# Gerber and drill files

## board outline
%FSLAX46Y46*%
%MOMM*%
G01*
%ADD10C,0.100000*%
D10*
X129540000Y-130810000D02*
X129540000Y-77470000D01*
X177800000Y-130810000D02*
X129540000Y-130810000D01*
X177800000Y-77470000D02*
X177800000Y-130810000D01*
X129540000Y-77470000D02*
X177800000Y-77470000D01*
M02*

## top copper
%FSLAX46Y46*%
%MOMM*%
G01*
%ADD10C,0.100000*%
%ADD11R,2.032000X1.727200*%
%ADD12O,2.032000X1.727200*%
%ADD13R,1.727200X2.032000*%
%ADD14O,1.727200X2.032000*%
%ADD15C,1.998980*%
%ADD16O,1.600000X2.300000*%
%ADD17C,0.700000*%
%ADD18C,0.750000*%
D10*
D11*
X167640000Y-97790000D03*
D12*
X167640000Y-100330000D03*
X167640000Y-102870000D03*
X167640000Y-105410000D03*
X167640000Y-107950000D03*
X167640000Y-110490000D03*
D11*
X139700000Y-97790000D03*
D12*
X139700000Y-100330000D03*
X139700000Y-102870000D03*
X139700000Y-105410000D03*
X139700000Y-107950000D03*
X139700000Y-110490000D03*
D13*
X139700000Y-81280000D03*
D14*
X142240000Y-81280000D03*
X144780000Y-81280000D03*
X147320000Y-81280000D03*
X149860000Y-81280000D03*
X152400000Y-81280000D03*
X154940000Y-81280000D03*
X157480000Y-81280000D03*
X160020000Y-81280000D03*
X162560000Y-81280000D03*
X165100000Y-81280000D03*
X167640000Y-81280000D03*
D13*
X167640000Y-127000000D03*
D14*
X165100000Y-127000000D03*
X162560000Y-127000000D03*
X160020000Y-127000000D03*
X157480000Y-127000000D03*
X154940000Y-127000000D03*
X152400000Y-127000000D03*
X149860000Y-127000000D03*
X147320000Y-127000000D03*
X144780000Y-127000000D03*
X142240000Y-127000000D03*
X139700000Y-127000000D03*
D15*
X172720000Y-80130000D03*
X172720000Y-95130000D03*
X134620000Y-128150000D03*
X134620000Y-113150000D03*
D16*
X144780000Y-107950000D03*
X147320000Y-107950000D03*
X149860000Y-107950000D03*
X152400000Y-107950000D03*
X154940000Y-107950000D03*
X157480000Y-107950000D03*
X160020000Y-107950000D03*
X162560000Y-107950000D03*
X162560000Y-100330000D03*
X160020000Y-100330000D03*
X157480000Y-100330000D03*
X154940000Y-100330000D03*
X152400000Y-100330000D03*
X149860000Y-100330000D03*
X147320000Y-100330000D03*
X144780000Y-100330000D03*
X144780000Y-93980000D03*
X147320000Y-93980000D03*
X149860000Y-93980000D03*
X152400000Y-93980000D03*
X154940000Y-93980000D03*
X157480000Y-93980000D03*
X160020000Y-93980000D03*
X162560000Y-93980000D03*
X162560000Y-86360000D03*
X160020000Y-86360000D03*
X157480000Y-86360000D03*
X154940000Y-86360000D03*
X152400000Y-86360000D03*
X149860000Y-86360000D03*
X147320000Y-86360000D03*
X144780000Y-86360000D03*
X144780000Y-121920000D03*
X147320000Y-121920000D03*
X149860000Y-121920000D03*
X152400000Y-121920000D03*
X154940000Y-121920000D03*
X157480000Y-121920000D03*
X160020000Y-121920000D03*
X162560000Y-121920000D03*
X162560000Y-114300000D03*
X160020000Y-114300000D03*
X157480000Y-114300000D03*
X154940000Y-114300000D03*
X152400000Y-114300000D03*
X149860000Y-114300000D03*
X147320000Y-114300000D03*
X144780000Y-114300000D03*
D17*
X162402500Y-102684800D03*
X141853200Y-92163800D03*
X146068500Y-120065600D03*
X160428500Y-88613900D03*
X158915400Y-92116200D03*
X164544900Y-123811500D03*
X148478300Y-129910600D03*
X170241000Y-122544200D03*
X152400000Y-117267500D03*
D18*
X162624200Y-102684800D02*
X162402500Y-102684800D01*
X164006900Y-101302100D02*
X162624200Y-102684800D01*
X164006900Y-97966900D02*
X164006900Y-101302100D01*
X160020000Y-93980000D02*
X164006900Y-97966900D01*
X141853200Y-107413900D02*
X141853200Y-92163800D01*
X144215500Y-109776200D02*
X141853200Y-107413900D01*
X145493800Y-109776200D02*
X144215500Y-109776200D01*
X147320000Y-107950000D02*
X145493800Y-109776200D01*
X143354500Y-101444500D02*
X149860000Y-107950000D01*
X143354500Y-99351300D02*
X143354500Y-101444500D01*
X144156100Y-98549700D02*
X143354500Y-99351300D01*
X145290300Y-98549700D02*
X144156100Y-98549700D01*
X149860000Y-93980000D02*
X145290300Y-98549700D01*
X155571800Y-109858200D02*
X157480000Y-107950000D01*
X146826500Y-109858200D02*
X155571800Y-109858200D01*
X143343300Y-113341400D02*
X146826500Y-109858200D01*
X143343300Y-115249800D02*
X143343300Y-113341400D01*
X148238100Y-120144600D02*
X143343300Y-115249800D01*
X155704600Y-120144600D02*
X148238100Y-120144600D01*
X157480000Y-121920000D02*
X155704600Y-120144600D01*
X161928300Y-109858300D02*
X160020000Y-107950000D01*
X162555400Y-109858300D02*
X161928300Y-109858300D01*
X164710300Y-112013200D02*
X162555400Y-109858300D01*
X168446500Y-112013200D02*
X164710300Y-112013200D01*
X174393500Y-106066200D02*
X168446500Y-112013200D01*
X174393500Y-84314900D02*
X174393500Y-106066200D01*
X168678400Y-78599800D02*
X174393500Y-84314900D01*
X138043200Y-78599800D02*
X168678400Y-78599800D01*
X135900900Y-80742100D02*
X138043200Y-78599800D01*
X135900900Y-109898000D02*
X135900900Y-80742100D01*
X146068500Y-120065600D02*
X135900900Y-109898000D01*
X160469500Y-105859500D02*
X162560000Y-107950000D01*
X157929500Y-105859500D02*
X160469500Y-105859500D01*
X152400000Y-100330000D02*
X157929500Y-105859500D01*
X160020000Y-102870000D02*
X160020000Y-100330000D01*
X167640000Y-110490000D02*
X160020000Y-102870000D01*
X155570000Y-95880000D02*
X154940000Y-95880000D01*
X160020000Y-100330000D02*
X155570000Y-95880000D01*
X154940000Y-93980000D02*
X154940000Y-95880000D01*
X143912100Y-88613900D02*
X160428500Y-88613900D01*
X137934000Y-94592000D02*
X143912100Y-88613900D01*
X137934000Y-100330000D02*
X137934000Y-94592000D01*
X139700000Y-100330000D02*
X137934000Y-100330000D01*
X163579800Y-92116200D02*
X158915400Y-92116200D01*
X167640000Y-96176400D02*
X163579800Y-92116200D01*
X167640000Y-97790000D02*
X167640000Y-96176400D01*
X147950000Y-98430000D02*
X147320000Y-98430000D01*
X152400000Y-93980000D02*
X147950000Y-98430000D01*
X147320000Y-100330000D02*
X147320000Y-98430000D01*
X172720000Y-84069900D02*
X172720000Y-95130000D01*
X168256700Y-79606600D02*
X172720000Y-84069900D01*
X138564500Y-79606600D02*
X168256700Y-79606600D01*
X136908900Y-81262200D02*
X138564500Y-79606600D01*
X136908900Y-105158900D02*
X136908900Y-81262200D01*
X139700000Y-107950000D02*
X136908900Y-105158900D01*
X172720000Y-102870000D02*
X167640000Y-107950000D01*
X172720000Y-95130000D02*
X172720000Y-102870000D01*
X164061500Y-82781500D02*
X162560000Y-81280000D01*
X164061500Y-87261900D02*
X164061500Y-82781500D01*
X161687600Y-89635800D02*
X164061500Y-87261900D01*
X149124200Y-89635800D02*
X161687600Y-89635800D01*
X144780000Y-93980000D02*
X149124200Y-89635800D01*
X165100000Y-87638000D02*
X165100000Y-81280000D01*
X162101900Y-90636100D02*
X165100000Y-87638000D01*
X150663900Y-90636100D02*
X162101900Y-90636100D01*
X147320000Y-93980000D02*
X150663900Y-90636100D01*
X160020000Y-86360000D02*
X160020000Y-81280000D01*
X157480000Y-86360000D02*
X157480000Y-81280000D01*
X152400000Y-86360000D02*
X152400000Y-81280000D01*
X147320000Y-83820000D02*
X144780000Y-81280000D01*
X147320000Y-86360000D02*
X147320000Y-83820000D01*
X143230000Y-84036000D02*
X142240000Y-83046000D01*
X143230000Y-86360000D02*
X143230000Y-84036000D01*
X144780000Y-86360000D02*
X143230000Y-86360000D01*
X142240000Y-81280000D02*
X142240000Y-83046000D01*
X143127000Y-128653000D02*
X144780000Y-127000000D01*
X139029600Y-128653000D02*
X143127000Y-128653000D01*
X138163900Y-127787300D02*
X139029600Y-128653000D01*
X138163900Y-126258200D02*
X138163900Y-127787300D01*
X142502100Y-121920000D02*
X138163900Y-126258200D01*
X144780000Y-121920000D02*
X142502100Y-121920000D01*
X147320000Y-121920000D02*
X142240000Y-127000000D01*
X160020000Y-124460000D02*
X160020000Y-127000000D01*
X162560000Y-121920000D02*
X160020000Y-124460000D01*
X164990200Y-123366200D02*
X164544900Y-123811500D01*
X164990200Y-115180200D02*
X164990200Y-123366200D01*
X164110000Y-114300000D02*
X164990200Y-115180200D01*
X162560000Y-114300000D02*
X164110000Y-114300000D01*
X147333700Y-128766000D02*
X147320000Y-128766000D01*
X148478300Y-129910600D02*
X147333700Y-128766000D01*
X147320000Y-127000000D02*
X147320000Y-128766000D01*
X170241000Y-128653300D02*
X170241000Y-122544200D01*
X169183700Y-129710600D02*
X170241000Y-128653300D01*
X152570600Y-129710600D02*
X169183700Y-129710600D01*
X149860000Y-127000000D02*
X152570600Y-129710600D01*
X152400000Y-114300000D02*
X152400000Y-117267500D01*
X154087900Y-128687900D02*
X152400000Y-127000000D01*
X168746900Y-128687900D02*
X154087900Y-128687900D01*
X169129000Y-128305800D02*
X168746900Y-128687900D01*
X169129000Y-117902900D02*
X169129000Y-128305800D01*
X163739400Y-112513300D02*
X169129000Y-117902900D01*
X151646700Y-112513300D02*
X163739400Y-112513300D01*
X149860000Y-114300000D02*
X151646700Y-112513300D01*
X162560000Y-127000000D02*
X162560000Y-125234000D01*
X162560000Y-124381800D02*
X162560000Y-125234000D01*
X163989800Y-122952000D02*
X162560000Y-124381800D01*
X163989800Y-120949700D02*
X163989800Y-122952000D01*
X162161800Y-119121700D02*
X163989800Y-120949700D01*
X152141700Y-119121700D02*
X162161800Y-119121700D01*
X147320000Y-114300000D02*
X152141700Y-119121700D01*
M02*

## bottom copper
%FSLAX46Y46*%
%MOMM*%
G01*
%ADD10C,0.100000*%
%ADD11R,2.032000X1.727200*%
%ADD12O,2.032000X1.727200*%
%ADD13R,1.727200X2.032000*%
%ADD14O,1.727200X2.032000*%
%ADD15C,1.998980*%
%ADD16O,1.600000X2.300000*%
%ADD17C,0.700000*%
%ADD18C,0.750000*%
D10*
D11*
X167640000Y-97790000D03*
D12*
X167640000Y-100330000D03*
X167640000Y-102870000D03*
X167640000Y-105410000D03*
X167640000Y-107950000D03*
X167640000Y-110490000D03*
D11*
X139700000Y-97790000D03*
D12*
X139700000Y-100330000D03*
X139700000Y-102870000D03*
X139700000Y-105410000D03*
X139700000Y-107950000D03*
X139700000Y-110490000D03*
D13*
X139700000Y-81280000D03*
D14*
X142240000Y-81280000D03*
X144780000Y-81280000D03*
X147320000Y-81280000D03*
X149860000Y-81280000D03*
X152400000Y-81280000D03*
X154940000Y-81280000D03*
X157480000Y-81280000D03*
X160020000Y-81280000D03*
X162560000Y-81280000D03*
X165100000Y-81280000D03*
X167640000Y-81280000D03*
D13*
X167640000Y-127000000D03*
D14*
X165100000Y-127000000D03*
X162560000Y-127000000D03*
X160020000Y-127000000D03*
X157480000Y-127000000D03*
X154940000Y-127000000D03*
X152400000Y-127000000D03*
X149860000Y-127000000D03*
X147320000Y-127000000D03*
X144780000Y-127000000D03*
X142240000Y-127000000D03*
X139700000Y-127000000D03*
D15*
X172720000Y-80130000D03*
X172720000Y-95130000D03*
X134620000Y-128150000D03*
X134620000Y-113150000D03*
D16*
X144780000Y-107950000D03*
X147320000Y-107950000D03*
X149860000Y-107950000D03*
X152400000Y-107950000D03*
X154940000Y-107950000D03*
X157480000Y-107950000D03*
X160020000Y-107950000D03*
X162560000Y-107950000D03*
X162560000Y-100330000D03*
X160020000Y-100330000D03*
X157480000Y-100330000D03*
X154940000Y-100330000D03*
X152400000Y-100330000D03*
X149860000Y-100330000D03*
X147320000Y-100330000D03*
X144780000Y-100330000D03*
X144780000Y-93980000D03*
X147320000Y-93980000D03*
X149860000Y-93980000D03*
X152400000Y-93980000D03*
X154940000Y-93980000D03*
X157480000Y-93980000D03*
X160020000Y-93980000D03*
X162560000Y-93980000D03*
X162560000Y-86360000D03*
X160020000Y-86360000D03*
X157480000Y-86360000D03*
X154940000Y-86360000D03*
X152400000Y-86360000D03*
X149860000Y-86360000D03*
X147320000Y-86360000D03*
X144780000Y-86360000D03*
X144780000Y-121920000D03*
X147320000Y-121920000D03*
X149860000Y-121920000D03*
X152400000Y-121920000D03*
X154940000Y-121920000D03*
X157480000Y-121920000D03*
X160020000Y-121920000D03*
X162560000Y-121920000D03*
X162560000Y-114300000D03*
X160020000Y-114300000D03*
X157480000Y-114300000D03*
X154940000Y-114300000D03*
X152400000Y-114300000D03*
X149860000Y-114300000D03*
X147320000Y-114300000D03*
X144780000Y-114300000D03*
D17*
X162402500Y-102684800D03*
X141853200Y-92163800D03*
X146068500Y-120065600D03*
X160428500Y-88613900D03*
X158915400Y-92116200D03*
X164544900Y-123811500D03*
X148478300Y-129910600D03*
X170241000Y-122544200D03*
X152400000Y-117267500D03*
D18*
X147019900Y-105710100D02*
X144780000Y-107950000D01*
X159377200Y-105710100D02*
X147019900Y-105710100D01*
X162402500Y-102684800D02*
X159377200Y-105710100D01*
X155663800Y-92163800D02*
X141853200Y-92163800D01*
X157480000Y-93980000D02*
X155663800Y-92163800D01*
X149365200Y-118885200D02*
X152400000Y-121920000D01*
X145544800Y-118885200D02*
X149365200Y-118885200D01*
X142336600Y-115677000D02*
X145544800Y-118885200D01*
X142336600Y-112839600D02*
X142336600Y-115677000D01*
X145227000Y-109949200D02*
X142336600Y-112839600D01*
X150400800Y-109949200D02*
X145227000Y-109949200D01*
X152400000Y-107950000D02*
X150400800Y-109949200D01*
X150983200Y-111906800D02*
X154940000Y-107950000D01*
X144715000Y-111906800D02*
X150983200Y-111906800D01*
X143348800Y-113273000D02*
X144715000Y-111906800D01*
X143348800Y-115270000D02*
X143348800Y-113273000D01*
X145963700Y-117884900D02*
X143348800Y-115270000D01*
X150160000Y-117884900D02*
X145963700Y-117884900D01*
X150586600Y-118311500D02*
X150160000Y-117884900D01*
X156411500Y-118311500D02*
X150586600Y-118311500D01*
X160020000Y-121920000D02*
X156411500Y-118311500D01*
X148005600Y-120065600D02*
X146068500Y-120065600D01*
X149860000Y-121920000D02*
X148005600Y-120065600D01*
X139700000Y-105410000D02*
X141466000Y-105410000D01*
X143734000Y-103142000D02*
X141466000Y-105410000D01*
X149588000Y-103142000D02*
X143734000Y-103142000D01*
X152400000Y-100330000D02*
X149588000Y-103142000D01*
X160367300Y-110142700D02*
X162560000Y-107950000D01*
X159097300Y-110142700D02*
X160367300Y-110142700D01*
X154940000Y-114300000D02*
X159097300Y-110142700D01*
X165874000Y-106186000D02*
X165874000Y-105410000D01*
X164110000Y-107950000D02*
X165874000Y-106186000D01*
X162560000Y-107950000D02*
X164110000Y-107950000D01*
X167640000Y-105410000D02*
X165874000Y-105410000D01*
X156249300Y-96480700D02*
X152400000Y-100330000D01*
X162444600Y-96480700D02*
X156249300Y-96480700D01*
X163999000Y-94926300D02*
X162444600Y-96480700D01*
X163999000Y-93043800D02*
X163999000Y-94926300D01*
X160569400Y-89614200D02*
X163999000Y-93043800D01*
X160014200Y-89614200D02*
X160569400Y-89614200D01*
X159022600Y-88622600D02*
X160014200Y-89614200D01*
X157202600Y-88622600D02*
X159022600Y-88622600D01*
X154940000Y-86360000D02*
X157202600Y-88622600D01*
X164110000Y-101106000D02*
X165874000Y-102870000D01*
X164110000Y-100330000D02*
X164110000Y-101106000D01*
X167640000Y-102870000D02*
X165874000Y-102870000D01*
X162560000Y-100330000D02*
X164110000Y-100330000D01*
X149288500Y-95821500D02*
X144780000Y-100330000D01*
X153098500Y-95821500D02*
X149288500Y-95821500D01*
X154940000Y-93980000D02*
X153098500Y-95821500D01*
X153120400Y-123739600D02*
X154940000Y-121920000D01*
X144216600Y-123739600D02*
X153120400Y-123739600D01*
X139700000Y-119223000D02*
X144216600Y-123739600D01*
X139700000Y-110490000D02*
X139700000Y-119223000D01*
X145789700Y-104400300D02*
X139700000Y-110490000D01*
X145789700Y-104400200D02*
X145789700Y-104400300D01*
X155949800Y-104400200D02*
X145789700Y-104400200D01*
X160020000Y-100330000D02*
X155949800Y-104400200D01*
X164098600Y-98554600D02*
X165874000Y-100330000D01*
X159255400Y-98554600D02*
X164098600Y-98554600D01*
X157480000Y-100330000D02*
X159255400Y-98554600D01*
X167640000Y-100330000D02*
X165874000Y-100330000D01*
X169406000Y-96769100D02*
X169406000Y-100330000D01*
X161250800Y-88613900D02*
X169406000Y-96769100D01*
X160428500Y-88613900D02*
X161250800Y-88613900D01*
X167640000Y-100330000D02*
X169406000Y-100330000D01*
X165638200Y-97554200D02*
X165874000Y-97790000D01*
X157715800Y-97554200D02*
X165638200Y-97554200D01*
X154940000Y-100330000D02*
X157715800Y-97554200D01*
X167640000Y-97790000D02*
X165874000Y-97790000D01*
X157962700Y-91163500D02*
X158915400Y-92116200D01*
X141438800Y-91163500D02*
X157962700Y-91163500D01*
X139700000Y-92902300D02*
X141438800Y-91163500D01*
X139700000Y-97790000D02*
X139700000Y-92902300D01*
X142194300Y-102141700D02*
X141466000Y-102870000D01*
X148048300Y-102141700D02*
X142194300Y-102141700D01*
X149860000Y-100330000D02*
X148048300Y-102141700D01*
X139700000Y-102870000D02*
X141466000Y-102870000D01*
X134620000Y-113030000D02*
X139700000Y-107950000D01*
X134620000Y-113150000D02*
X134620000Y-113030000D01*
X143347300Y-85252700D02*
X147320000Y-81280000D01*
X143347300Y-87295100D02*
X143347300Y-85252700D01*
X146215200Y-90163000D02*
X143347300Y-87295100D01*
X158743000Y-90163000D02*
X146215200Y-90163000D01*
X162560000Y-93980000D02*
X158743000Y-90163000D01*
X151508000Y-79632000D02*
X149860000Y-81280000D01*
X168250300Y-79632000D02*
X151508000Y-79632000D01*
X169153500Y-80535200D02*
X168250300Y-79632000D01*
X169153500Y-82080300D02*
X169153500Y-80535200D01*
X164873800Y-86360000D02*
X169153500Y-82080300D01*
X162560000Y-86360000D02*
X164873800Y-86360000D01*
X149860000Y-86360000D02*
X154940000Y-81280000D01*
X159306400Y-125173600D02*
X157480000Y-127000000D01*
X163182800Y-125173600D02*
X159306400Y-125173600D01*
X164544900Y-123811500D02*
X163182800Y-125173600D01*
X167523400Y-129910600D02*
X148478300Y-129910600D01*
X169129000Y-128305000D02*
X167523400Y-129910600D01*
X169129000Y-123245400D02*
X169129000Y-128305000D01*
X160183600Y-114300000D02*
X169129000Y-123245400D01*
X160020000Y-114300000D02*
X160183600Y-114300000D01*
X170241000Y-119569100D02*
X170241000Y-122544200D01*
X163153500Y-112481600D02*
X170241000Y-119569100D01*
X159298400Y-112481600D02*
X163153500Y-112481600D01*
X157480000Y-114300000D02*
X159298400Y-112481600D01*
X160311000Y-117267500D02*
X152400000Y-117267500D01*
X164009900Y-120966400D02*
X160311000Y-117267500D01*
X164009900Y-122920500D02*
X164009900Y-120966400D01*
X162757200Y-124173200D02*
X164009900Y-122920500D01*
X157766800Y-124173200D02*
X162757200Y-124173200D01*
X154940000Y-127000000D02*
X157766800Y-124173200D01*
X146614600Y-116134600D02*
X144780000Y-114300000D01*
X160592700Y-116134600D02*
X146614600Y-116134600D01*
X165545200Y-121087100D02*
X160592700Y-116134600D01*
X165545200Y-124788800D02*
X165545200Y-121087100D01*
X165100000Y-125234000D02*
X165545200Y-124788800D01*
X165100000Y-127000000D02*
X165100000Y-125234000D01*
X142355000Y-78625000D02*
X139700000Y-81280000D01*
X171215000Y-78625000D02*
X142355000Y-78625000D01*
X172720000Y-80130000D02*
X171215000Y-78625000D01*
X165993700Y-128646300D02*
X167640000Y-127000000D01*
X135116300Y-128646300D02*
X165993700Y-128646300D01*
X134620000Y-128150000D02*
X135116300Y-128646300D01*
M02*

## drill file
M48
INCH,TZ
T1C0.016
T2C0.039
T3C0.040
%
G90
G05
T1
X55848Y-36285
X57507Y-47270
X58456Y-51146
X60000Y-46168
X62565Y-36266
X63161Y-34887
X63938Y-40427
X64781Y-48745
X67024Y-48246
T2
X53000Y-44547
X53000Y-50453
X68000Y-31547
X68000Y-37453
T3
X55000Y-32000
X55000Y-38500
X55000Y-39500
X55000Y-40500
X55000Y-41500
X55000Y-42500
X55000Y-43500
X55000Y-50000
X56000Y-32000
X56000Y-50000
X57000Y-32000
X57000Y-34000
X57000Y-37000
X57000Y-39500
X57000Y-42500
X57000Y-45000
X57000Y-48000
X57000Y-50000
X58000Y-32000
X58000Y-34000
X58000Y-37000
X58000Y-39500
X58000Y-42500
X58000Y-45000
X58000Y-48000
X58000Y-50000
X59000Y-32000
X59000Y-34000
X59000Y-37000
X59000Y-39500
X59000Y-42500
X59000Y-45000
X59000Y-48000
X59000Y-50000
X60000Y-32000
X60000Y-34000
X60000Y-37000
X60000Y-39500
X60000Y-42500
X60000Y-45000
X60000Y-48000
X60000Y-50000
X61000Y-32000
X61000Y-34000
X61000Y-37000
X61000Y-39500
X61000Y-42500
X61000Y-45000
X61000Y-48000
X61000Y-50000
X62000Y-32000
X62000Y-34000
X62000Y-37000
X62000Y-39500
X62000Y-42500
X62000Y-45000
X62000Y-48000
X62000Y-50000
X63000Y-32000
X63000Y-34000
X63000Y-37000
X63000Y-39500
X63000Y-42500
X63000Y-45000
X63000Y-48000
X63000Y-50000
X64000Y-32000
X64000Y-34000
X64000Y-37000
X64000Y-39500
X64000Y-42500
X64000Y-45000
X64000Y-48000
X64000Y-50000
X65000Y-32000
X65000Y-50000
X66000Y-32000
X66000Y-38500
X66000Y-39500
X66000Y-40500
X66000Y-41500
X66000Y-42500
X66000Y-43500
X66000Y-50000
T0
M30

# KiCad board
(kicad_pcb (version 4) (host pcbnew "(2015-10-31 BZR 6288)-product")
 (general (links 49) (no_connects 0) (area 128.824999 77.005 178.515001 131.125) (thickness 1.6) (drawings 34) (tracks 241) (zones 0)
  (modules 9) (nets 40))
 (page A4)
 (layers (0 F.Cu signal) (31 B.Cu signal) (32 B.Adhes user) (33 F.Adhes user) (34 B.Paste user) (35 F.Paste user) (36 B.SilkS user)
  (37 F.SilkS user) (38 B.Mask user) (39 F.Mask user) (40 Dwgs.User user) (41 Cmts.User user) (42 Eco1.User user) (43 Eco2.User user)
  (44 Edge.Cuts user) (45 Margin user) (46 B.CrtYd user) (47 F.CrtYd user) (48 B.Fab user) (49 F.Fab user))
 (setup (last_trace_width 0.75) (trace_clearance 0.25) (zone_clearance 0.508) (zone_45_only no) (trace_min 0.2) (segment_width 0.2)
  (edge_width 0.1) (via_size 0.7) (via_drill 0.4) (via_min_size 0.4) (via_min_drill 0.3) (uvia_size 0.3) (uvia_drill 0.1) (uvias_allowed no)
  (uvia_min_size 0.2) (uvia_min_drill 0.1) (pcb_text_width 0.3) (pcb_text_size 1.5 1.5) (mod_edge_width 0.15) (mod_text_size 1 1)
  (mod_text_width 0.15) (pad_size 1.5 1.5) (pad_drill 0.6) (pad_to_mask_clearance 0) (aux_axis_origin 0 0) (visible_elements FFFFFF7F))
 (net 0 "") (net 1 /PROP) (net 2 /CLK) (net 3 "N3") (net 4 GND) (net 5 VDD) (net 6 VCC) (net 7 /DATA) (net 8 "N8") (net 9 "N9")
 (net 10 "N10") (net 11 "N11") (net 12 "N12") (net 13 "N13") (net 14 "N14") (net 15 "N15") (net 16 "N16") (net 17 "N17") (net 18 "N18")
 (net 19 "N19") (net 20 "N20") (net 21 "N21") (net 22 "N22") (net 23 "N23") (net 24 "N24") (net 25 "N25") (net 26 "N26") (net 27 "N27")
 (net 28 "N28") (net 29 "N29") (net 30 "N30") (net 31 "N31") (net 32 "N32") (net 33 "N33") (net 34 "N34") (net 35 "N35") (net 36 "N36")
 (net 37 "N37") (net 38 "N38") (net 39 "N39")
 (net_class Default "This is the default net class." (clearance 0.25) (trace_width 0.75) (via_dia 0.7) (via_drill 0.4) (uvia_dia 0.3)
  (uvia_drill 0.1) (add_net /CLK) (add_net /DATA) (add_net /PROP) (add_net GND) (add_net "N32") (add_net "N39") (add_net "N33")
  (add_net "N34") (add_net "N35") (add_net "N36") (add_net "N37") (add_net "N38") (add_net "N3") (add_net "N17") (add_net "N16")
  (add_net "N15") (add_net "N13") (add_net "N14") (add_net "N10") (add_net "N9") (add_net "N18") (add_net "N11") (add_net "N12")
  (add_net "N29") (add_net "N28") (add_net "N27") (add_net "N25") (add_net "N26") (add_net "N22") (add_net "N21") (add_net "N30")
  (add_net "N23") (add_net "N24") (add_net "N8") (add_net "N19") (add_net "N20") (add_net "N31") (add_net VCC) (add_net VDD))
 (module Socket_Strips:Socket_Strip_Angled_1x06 (layer B.Cu) (at 167.64 97.79 270)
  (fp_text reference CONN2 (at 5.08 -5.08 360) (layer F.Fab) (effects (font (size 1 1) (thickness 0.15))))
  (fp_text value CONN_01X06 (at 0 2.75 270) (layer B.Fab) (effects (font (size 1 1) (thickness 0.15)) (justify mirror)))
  (pad 1 thru_hole rect (at 0 0 270) (size 1.7272 2.032) (drill 1.016) (layers *.Cu *.Mask B.SilkS) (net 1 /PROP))
  (pad 2 thru_hole oval (at 2.54 0 270) (size 1.7272 2.032) (drill 1.016) (layers *.Cu *.Mask B.SilkS) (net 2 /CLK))
  (pad 3 thru_hole oval (at 5.08 0 270) (size 1.7272 2.032) (drill 1.016) (layers *.Cu *.Mask B.SilkS) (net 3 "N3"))
  (pad 4 thru_hole oval (at 7.62 0 270) (size 1.7272 2.032) (drill 1.016) (layers *.Cu *.Mask B.SilkS) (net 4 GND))
  (pad 5 thru_hole oval (at 10.16 0 270) (size 1.7272 2.032) (drill 1.016) (layers *.Cu *.Mask B.SilkS) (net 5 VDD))
  (pad 6 thru_hole oval (at 12.7 0 270) (size 1.7272 2.032) (drill 1.016) (layers *.Cu *.Mask B.SilkS) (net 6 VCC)))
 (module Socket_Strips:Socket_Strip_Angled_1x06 (layer F.Cu) (at 139.7 97.79 270)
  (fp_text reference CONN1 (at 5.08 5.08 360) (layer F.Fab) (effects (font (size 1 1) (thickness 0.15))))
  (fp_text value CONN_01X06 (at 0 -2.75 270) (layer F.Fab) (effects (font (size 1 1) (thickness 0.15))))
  (pad 1 thru_hole rect (at 0 0 270) (size 1.7272 2.032) (drill 1.016) (layers *.Cu *.Mask F.SilkS) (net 1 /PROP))
  (pad 2 thru_hole oval (at 2.54 0 270) (size 1.7272 2.032) (drill 1.016) (layers *.Cu *.Mask F.SilkS) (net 2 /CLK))
  (pad 3 thru_hole oval (at 5.08 0 270) (size 1.7272 2.032) (drill 1.016) (layers *.Cu *.Mask F.SilkS) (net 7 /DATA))
  (pad 4 thru_hole oval (at 7.62 0 270) (size 1.7272 2.032) (drill 1.016) (layers *.Cu *.Mask F.SilkS) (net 4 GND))
  (pad 5 thru_hole oval (at 10.16 0 270) (size 1.7272 2.032) (drill 1.016) (layers *.Cu *.Mask F.SilkS) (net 5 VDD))
  (pad 6 thru_hole oval (at 12.7 0 270) (size 1.7272 2.032) (drill 1.016) (layers *.Cu *.Mask F.SilkS) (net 6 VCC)))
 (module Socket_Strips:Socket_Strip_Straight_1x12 (layer F.Cu) (at 139.7 81.28)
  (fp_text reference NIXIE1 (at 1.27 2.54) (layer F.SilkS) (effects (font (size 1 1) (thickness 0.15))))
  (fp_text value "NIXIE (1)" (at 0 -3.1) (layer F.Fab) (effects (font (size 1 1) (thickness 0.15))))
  (pad 1 thru_hole rect (at 0 0) (size 1.7272 2.032) (drill 1.016) (layers *.Cu *.Mask F.SilkS) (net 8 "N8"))
  (pad 2 thru_hole oval (at 2.54 0) (size 1.7272 2.032) (drill 1.016) (layers *.Cu *.Mask F.SilkS) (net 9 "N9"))
  (pad 3 thru_hole oval (at 5.08 0) (size 1.7272 2.032) (drill 1.016) (layers *.Cu *.Mask F.SilkS) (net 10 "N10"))
  (pad 4 thru_hole oval (at 7.62 0) (size 1.7272 2.032) (drill 1.016) (layers *.Cu *.Mask F.SilkS) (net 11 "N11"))
  (pad 5 thru_hole oval (at 10.16 0) (size 1.7272 2.032) (drill 1.016) (layers *.Cu *.Mask F.SilkS) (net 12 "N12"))
  (pad 6 thru_hole oval (at 12.7 0) (size 1.7272 2.032) (drill 1.016) (layers *.Cu *.Mask F.SilkS) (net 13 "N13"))
  (pad 7 thru_hole oval (at 15.24 0) (size 1.7272 2.032) (drill 1.016) (layers *.Cu *.Mask F.SilkS) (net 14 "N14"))
  (pad 8 thru_hole oval (at 17.78 0) (size 1.7272 2.032) (drill 1.016) (layers *.Cu *.Mask F.SilkS) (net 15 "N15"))
  (pad 9 thru_hole oval (at 20.32 0) (size 1.7272 2.032) (drill 1.016) (layers *.Cu *.Mask F.SilkS) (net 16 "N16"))
  (pad 10 thru_hole oval (at 22.86 0) (size 1.7272 2.032) (drill 1.016) (layers *.Cu *.Mask F.SilkS) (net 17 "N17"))
  (pad 11 thru_hole oval (at 25.4 0) (size 1.7272 2.032) (drill 1.016) (layers *.Cu *.Mask F.SilkS) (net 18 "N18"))
  (pad 12 thru_hole oval (at 27.94 0) (size 1.7272 2.032) (drill 1.016) (layers *.Cu *.Mask F.SilkS) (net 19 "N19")))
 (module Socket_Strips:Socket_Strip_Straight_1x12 (layer F.Cu) (at 167.64 127 180)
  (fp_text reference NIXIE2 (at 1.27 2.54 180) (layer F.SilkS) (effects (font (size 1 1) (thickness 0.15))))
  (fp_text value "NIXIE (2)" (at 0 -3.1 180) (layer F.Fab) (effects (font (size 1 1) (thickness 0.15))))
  (pad 1 thru_hole rect (at 0 0 180) (size 1.7272 2.032) (drill 1.016) (layers *.Cu *.Mask F.SilkS) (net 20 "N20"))
  (pad 2 thru_hole oval (at 2.54 0 180) (size 1.7272 2.032) (drill 1.016) (layers *.Cu *.Mask F.SilkS) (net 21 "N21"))
  (pad 3 thru_hole oval (at 5.08 0 180) (size 1.7272 2.032) (drill 1.016) (layers *.Cu *.Mask F.SilkS) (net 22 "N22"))
  (pad 4 thru_hole oval (at 7.62 0 180) (size 1.7272 2.032) (drill 1.016) (layers *.Cu *.Mask F.SilkS) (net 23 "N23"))
  (pad 5 thru_hole oval (at 10.16 0 180) (size 1.7272 2.032) (drill 1.016) (layers *.Cu *.Mask F.SilkS) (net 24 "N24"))
  (pad 6 thru_hole oval (at 12.7 0 180) (size 1.7272 2.032) (drill 1.016) (layers *.Cu *.Mask F.SilkS) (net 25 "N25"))
  (pad 7 thru_hole oval (at 15.24 0 180) (size 1.7272 2.032) (drill 1.016) (layers *.Cu *.Mask F.SilkS) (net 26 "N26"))
  (pad 8 thru_hole oval (at 17.78 0 180) (size 1.7272 2.032) (drill 1.016) (layers *.Cu *.Mask F.SilkS) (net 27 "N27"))
  (pad 9 thru_hole oval (at 20.32 0 180) (size 1.7272 2.032) (drill 1.016) (layers *.Cu *.Mask F.SilkS) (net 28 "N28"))
  (pad 10 thru_hole oval (at 22.86 0 180) (size 1.7272 2.032) (drill 1.016) (layers *.Cu *.Mask F.SilkS) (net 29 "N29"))
  (pad 11 thru_hole oval (at 25.4 0 180) (size 1.7272 2.032) (drill 1.016) (layers *.Cu *.Mask F.SilkS) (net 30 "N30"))
  (pad 12 thru_hole oval (at 27.94 0 180) (size 1.7272 2.032) (drill 1.016) (layers *.Cu *.Mask F.SilkS) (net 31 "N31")))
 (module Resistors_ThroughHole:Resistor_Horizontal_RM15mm (layer F.Cu) (at 172.72 87.63 270)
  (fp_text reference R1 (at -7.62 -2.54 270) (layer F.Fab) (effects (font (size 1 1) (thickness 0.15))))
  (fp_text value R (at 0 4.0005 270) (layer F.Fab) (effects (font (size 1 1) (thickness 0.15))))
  (pad 1 thru_hole circle (at -7.5 0 270) (size 1.99898 1.99898) (drill 1.00076) (layers *.Cu *.SilkS *.Mask) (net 8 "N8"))
  (pad 2 thru_hole circle (at 7.5 0 270) (size 1.99898 1.99898) (drill 1.00076) (layers *.Cu *.SilkS *.Mask) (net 5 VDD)))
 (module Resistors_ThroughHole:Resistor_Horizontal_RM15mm (layer F.Cu) (at 134.62 120.65 90)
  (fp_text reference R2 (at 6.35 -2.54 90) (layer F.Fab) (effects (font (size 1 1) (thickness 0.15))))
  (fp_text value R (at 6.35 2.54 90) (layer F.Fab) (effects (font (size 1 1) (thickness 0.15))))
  (pad 1 thru_hole circle (at -7.5 0 90) (size 1.99898 1.99898) (drill 1.00076) (layers *.Cu *.SilkS *.Mask) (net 20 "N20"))
  (pad 2 thru_hole circle (at 7.5 0 90) (size 1.99898 1.99898) (drill 1.00076) (layers *.Cu *.SilkS *.Mask) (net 5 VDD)))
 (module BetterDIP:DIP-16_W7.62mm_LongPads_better (layer F.Cu) (at 144.78 107.95 90)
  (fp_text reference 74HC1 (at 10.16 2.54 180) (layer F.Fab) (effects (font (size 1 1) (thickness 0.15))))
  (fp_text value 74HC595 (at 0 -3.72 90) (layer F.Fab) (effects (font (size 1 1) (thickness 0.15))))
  (pad 1 thru_hole oval (at 0 0 90) (size 2.3 1.6) (drill 1.016) (layers *.Cu *.Mask F.SilkS) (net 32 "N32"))
  (pad 2 thru_hole oval (at 0 2.54 90) (size 2.3 1.6) (drill 1.016) (layers *.Cu *.Mask F.SilkS) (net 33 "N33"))
  (pad 3 thru_hole oval (at 0 5.08 90) (size 2.3 1.6) (drill 1.016) (layers *.Cu *.Mask F.SilkS) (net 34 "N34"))
  (pad 4 thru_hole oval (at 0 7.62 90) (size 2.3 1.6) (drill 1.016) (layers *.Cu *.Mask F.SilkS) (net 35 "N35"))
  (pad 5 thru_hole oval (at 0 10.16 90) (size 2.3 1.6) (drill 1.016) (layers *.Cu *.Mask F.SilkS) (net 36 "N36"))
  (pad 6 thru_hole oval (at 0 12.7 90) (size 2.3 1.6) (drill 1.016) (layers *.Cu *.Mask F.SilkS) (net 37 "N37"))
  (pad 7 thru_hole oval (at 0 15.24 90) (size 2.3 1.6) (drill 1.016) (layers *.Cu *.Mask F.SilkS) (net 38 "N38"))
  (pad 8 thru_hole oval (at 0 17.78 90) (size 2.3 1.6) (drill 1.016) (layers *.Cu *.Mask F.SilkS) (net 4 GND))
  (pad 9 thru_hole oval (at 7.62 17.78 90) (size 2.3 1.6) (drill 1.016) (layers *.Cu *.Mask F.SilkS) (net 3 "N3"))
  (pad 10 thru_hole oval (at 7.62 15.24 90) (size 2.3 1.6) (drill 1.016) (layers *.Cu *.Mask F.SilkS) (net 6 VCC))
  (pad 11 thru_hole oval (at 7.62 12.7 90) (size 2.3 1.6) (drill 1.016) (layers *.Cu *.Mask F.SilkS) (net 2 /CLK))
  (pad 12 thru_hole oval (at 7.62 10.16 90) (size 2.3 1.6) (drill 1.016) (layers *.Cu *.Mask F.SilkS) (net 1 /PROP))
  (pad 13 thru_hole oval (at 7.62 7.62 90) (size 2.3 1.6) (drill 1.016) (layers *.Cu *.Mask F.SilkS) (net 4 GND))
  (pad 14 thru_hole oval (at 7.62 5.08 90) (size 2.3 1.6) (drill 1.016) (layers *.Cu *.Mask F.SilkS) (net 7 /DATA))
  (pad 15 thru_hole oval (at 7.62 2.54 90) (size 2.3 1.6) (drill 1.016) (layers *.Cu *.Mask F.SilkS) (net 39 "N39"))
  (pad 16 thru_hole oval (at 7.62 0 90) (size 2.3 1.6) (drill 1.016) (layers *.Cu *.Mask F.SilkS) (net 6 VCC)))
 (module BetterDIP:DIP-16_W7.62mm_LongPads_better (layer F.Cu) (at 144.78 93.98 90)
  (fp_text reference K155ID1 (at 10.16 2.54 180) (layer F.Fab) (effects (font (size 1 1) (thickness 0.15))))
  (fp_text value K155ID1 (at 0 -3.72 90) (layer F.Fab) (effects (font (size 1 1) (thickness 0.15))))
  (pad 1 thru_hole oval (at 0 0 90) (size 2.3 1.6) (drill 1.016) (layers *.Cu *.Mask F.SilkS) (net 17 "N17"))
  (pad 2 thru_hole oval (at 0 2.54 90) (size 2.3 1.6) (drill 1.016) (layers *.Cu *.Mask F.SilkS) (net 18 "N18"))
  (pad 3 thru_hole oval (at 0 5.08 90) (size 2.3 1.6) (drill 1.016) (layers *.Cu *.Mask F.SilkS) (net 34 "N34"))
  (pad 4 thru_hole oval (at 0 7.62 90) (size 2.3 1.6) (drill 1.016) (layers *.Cu *.Mask F.SilkS) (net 39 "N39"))
  (pad 5 thru_hole oval (at 0 10.16 90) (size 2.3 1.6) (drill 1.016) (layers *.Cu *.Mask F.SilkS) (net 6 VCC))
  (pad 6 thru_hole oval (at 0 12.7 90) (size 2.3 1.6) (drill 1.016) (layers *.Cu *.Mask F.SilkS) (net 33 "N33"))
  (pad 7 thru_hole oval (at 0 15.24 90) (size 2.3 1.6) (drill 1.016) (layers *.Cu *.Mask F.SilkS) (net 32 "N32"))
  (pad 8 thru_hole oval (at 0 17.78 90) (size 2.3 1.6) (drill 1.016) (layers *.Cu *.Mask F.SilkS) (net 11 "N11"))
  (pad 9 thru_hole oval (at 7.62 17.78 90) (size 2.3 1.6) (drill 1.016) (layers *.Cu *.Mask F.SilkS) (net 12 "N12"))
  (pad 10 thru_hole oval (at 7.62 15.24 90) (size 2.3 1.6) (drill 1.016) (layers *.Cu *.Mask F.SilkS) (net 16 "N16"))
  (pad 11 thru_hole oval (at 7.62 12.7 90) (size 2.3 1.6) (drill 1.016) (layers *.Cu *.Mask F.SilkS) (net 15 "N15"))
  (pad 12 thru_hole oval (at 7.62 10.16 90) (size 2.3 1.6) (drill 1.016) (layers *.Cu *.Mask F.SilkS) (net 4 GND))
  (pad 13 thru_hole oval (at 7.62 7.62 90) (size 2.3 1.6) (drill 1.016) (layers *.Cu *.Mask F.SilkS) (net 13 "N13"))
  (pad 14 thru_hole oval (at 7.62 5.08 90) (size 2.3 1.6) (drill 1.016) (layers *.Cu *.Mask F.SilkS) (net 14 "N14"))
  (pad 15 thru_hole oval (at 7.62 2.54 90) (size 2.3 1.6) (drill 1.016) (layers *.Cu *.Mask F.SilkS) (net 10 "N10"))
  (pad 16 thru_hole oval (at 7.62 0 90) (size 2.3 1.6) (drill 1.016) (layers *.Cu *.Mask F.SilkS) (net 9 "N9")))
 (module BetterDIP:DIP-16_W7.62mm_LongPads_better (layer F.Cu) (at 144.78 121.92 90)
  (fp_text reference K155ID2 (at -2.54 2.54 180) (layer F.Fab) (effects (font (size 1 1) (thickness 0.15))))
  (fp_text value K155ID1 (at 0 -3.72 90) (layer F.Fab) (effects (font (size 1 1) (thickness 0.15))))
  (pad 1 thru_hole oval (at 0 0 90) (size 2.3 1.6) (drill 1.016) (layers *.Cu *.Mask F.SilkS) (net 29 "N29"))
  (pad 2 thru_hole oval (at 0 2.54 90) (size 2.3 1.6) (drill 1.016) (layers *.Cu *.Mask F.SilkS) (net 30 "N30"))
  (pad 3 thru_hole oval (at 0 5.08 90) (size 2.3 1.6) (drill 1.016) (layers *.Cu *.Mask F.SilkS) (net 38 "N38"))
  (pad 4 thru_hole oval (at 0 7.62 90) (size 2.3 1.6) (drill 1.016) (layers *.Cu *.Mask F.SilkS) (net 35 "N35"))
  (pad 5 thru_hole oval (at 0 10.16 90) (size 2.3 1.6) (drill 1.016) (layers *.Cu *.Mask F.SilkS) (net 6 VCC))
  (pad 6 thru_hole oval (at 0 12.7 90) (size 2.3 1.6) (drill 1.016) (layers *.Cu *.Mask F.SilkS) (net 37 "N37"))
  (pad 7 thru_hole oval (at 0 15.24 90) (size 2.3 1.6) (drill 1.016) (layers *.Cu *.Mask F.SilkS) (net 36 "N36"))
  (pad 8 thru_hole oval (at 0 17.78 90) (size 2.3 1.6) (drill 1.016) (layers *.Cu *.Mask F.SilkS) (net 23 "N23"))
  (pad 9 thru_hole oval (at 7.62 17.78 90) (size 2.3 1.6) (drill 1.016) (layers *.Cu *.Mask F.SilkS) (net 24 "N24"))
  (pad 10 thru_hole oval (at 7.62 15.24 90) (size 2.3 1.6) (drill 1.016) (layers *.Cu *.Mask F.SilkS) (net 28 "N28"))
  (pad 11 thru_hole oval (at 7.62 12.7 90) (size 2.3 1.6) (drill 1.016) (layers *.Cu *.Mask F.SilkS) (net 27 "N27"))
  (pad 12 thru_hole oval (at 7.62 10.16 90) (size 2.3 1.6) (drill 1.016) (layers *.Cu *.Mask F.SilkS) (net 4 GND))
  (pad 13 thru_hole oval (at 7.62 7.62 90) (size 2.3 1.6) (drill 1.016) (layers *.Cu *.Mask F.SilkS) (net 25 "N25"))
  (pad 14 thru_hole oval (at 7.62 5.08 90) (size 2.3 1.6) (drill 1.016) (layers *.Cu *.Mask F.SilkS) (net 26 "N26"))
  (pad 15 thru_hole oval (at 7.62 2.54 90) (size 2.3 1.6) (drill 1.016) (layers *.Cu *.Mask F.SilkS) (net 22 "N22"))
  (pad 16 thru_hole oval (at 7.62 0 90) (size 2.3 1.6) (drill 1.016) (layers *.Cu *.Mask F.SilkS) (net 21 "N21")))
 (gr_line (start 129.54 130.81) (end 129.54 77.47) (angle 90) (layer Edge.Cuts) (width 0.1))
 (gr_line (start 177.8 130.81) (end 129.54 130.81) (angle 90) (layer Edge.Cuts) (width 0.1))
 (gr_line (start 177.8 77.47) (end 177.8 130.81) (angle 90) (layer Edge.Cuts) (width 0.1))
 (gr_line (start 129.54 77.47) (end 177.8 77.47) (angle 90) (layer Edge.Cuts) (width 0.1))
 (via (at 162.4025 102.6848) (size 0.7) (layers F.Cu B.Cu) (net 32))
 (segment (start 162.6242 102.6848) (end 162.4025 102.6848) (width 0.75) (layer F.Cu) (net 32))
 (segment (start 164.0069 101.3021) (end 162.6242 102.6848) (width 0.75) (layer F.Cu) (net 32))
 (segment (start 164.0069 97.9669) (end 164.0069 101.3021) (width 0.75) (layer F.Cu) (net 32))
 (segment (start 160.02 93.98) (end 164.0069 97.9669) (width 0.75) (layer F.Cu) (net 32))
 (segment (start 147.0199 105.7101) (end 144.78 107.95) (width 0.75) (layer B.Cu) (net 32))
 (segment (start 159.3772 105.7101) (end 147.0199 105.7101) (width 0.75) (layer B.Cu) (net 32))
 (segment (start 162.4025 102.6848) (end 159.3772 105.7101) (width 0.75) (layer B.Cu) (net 32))
 (via (at 141.8532 92.1638) (size 0.7) (layers F.Cu B.Cu) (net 33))
 (segment (start 155.6638 92.1638) (end 141.8532 92.1638) (width 0.75) (layer B.Cu) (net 33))
 (segment (start 157.48 93.98) (end 155.6638 92.1638) (width 0.75) (layer B.Cu) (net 33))
 (segment (start 141.8532 107.4139) (end 141.8532 92.1638) (width 0.75) (layer F.Cu) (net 33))
 (segment (start 144.2155 109.7762) (end 141.8532 107.4139) (width 0.75) (layer F.Cu) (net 33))
 (segment (start 145.4938 109.7762) (end 144.2155 109.7762) (width 0.75) (layer F.Cu) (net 33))
 (segment (start 147.32 107.95) (end 145.4938 109.7762) (width 0.75) (layer F.Cu) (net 33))
 (segment (start 143.3545 101.4445) (end 149.86 107.95) (width 0.75) (layer F.Cu) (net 34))
 (segment (start 143.3545 99.3513) (end 143.3545 101.4445) (width 0.75) (layer F.Cu) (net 34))
 (segment (start 144.1561 98.5497) (end 143.3545 99.3513) (width 0.75) (layer F.Cu) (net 34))
 (segment (start 145.2903 98.5497) (end 144.1561 98.5497) (width 0.75) (layer F.Cu) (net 34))
 (segment (start 149.86 93.98) (end 145.2903 98.5497) (width 0.75) (layer F.Cu) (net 34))
 (segment (start 149.3652 118.8852) (end 152.4 121.92) (width 0.75) (layer B.Cu) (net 35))
 (segment (start 145.5448 118.8852) (end 149.3652 118.8852) (width 0.75) (layer B.Cu) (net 35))
 (segment (start 142.3366 115.677) (end 145.5448 118.8852) (width 0.75) (layer B.Cu) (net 35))
 (segment (start 142.3366 112.8396) (end 142.3366 115.677) (width 0.75) (layer B.Cu) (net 35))
 (segment (start 145.227 109.9492) (end 142.3366 112.8396) (width 0.75) (layer B.Cu) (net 35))
 (segment (start 150.4008 109.9492) (end 145.227 109.9492) (width 0.75) (layer B.Cu) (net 35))
 (segment (start 152.4 107.95) (end 150.4008 109.9492) (width 0.75) (layer B.Cu) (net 35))
 (segment (start 150.9832 111.9068) (end 154.94 107.95) (width 0.75) (layer B.Cu) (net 36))
 (segment (start 144.715 111.9068) (end 150.9832 111.9068) (width 0.75) (layer B.Cu) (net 36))
 (segment (start 143.3488 113.273) (end 144.715 111.9068) (width 0.75) (layer B.Cu) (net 36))
 (segment (start 143.3488 115.27) (end 143.3488 113.273) (width 0.75) (layer B.Cu) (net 36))
 (segment (start 145.9637 117.8849) (end 143.3488 115.27) (width 0.75) (layer B.Cu) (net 36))
 (segment (start 150.16 117.8849) (end 145.9637 117.8849) (width 0.75) (layer B.Cu) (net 36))
 (segment (start 150.5866 118.3115) (end 150.16 117.8849) (width 0.75) (layer B.Cu) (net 36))
 (segment (start 156.4115 118.3115) (end 150.5866 118.3115) (width 0.75) (layer B.Cu) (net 36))
 (segment (start 160.02 121.92) (end 156.4115 118.3115) (width 0.75) (layer B.Cu) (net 36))
 (segment (start 155.5718 109.8582) (end 157.48 107.95) (width 0.75) (layer F.Cu) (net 37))
 (segment (start 146.8265 109.8582) (end 155.5718 109.8582) (width 0.75) (layer F.Cu) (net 37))
 (segment (start 143.3433 113.3414) (end 146.8265 109.8582) (width 0.75) (layer F.Cu) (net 37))
 (segment (start 143.3433 115.2498) (end 143.3433 113.3414) (width 0.75) (layer F.Cu) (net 37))
 (segment (start 148.2381 120.1446) (end 143.3433 115.2498) (width 0.75) (layer F.Cu) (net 37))
 (segment (start 155.7046 120.1446) (end 148.2381 120.1446) (width 0.75) (layer F.Cu) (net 37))
 (segment (start 157.48 121.92) (end 155.7046 120.1446) (width 0.75) (layer F.Cu) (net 37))
 (via (at 146.0685 120.0656) (size 0.7) (layers F.Cu B.Cu) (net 38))
 (segment (start 148.0056 120.0656) (end 146.0685 120.0656) (width 0.75) (layer B.Cu) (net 38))
 (segment (start 149.86 121.92) (end 148.0056 120.0656) (width 0.75) (layer B.Cu) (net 38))
 (segment (start 161.9283 109.8583) (end 160.02 107.95) (width 0.75) (layer F.Cu) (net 38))
 (segment (start 162.5554 109.8583) (end 161.9283 109.8583) (width 0.75) (layer F.Cu) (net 38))
 (segment (start 164.7103 112.0132) (end 162.5554 109.8583) (width 0.75) (layer F.Cu) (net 38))
 (segment (start 168.4465 112.0132) (end 164.7103 112.0132) (width 0.75) (layer F.Cu) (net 38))
 (segment (start 174.3935 106.0662) (end 168.4465 112.0132) (width 0.75) (layer F.Cu) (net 38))
 (segment (start 174.3935 84.3149) (end 174.3935 106.0662) (width 0.75) (layer F.Cu) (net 38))
 (segment (start 168.6784 78.5998) (end 174.3935 84.3149) (width 0.75) (layer F.Cu) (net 38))
 (segment (start 138.0432 78.5998) (end 168.6784 78.5998) (width 0.75) (layer F.Cu) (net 38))
 (segment (start 135.9009 80.7421) (end 138.0432 78.5998) (width 0.75) (layer F.Cu) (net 38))
 (segment (start 135.9009 109.898) (end 135.9009 80.7421) (width 0.75) (layer F.Cu) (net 38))
 (segment (start 146.0685 120.0656) (end 135.9009 109.898) (width 0.75) (layer F.Cu) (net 38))
 (segment (start 139.7 105.41) (end 141.466 105.41) (width 0.75) (layer B.Cu) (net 4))
 (segment (start 160.4695 105.8595) (end 162.56 107.95) (width 0.75) (layer F.Cu) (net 4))
 (segment (start 157.9295 105.8595) (end 160.4695 105.8595) (width 0.75) (layer F.Cu) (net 4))
 (segment (start 152.4 100.33) (end 157.9295 105.8595) (width 0.75) (layer F.Cu) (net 4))
 (segment (start 143.734 103.142) (end 141.466 105.41) (width 0.75) (layer B.Cu) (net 4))
 (segment (start 149.588 103.142) (end 143.734 103.142) (width 0.75) (layer B.Cu) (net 4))
 (segment (start 152.4 100.33) (end 149.588 103.142) (width 0.75) (layer B.Cu) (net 4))
 (segment (start 160.3673 110.1427) (end 162.56 107.95) (width 0.75) (layer B.Cu) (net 4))
 (segment (start 159.0973 110.1427) (end 160.3673 110.1427) (width 0.75) (layer B.Cu) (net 4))
 (segment (start 154.94 114.3) (end 159.0973 110.1427) (width 0.75) (layer B.Cu) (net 4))
 (segment (start 165.874 106.186) (end 165.874 105.41) (width 0.75) (layer B.Cu) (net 4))
 (segment (start 164.11 107.95) (end 165.874 106.186) (width 0.75) (layer B.Cu) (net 4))
 (segment (start 162.56 107.95) (end 164.11 107.95) (width 0.75) (layer B.Cu) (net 4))
 (segment (start 167.64 105.41) (end 165.874 105.41) (width 0.75) (layer B.Cu) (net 4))
 (segment (start 156.2493 96.4807) (end 152.4 100.33) (width 0.75) (layer B.Cu) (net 4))
 (segment (start 162.4446 96.4807) (end 156.2493 96.4807) (width 0.75) (layer B.Cu) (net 4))
 (segment (start 163.999 94.9263) (end 162.4446 96.4807) (width 0.75) (layer B.Cu) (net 4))
 (segment (start 163.999 93.0438) (end 163.999 94.9263) (width 0.75) (layer B.Cu) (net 4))
 (segment (start 160.5694 89.6142) (end 163.999 93.0438) (width 0.75) (layer B.Cu) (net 4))
 (segment (start 160.0142 89.6142) (end 160.5694 89.6142) (width 0.75) (layer B.Cu) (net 4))
 (segment (start 159.0226 88.6226) (end 160.0142 89.6142) (width 0.75) (layer B.Cu) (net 4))
 (segment (start 157.2026 88.6226) (end 159.0226 88.6226) (width 0.75) (layer B.Cu) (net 4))
 (segment (start 154.94 86.36) (end 157.2026 88.6226) (width 0.75) (layer B.Cu) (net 4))
 (segment (start 164.11 101.106) (end 165.874 102.87) (width 0.75) (layer B.Cu) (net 3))
 (segment (start 164.11 100.33) (end 164.11 101.106) (width 0.75) (layer B.Cu) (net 3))
 (segment (start 167.64 102.87) (end 165.874 102.87) (width 0.75) (layer B.Cu) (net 3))
 (segment (start 162.56 100.33) (end 164.11 100.33) (width 0.75) (layer B.Cu) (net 3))
 (segment (start 149.2885 95.8215) (end 144.78 100.33) (width 0.75) (layer B.Cu) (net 6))
 (segment (start 153.0985 95.8215) (end 149.2885 95.8215) (width 0.75) (layer B.Cu) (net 6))
 (segment (start 154.94 93.98) (end 153.0985 95.8215) (width 0.75) (layer B.Cu) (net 6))
 (segment (start 160.02 102.87) (end 160.02 100.33) (width 0.75) (layer F.Cu) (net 6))
 (segment (start 167.64 110.49) (end 160.02 102.87) (width 0.75) (layer F.Cu) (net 6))
 (segment (start 155.57 95.88) (end 154.94 95.88) (width 0.75) (layer F.Cu) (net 6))
 (segment (start 160.02 100.33) (end 155.57 95.88) (width 0.75) (layer F.Cu) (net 6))
 (segment (start 154.94 93.98) (end 154.94 95.88) (width 0.75) (layer F.Cu) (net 6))
 (segment (start 153.1204 123.7396) (end 154.94 121.92) (width 0.75) (layer B.Cu) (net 6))
 (segment (start 144.2166 123.7396) (end 153.1204 123.7396) (width 0.75) (layer B.Cu) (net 6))
 (segment (start 139.7 119.223) (end 144.2166 123.7396) (width 0.75) (layer B.Cu) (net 6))
 (segment (start 139.7 110.49) (end 139.7 119.223) (width 0.75) (layer B.Cu) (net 6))
 (segment (start 145.7897 104.4003) (end 139.7 110.49) (width 0.75) (layer B.Cu) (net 6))
 (segment (start 145.7897 104.4002) (end 145.7897 104.4003) (width 0.75) (layer B.Cu) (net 6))
 (segment (start 155.9498 104.4002) (end 145.7897 104.4002) (width 0.75) (layer B.Cu) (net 6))
 (segment (start 160.02 100.33) (end 155.9498 104.4002) (width 0.75) (layer B.Cu) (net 6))
 (via (at 160.4285 88.6139) (size 0.7) (layers F.Cu B.Cu) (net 2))
 (segment (start 164.0986 98.5546) (end 165.874 100.33) (width 0.75) (layer B.Cu) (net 2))
 (segment (start 159.2554 98.5546) (end 164.0986 98.5546) (width 0.75) (layer B.Cu) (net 2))
 (segment (start 157.48 100.33) (end 159.2554 98.5546) (width 0.75) (layer B.Cu) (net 2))
 (segment (start 167.64 100.33) (end 165.874 100.33) (width 0.75) (layer B.Cu) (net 2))
 (segment (start 143.9121 88.6139) (end 160.4285 88.6139) (width 0.75) (layer F.Cu) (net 2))
 (segment (start 137.934 94.592) (end 143.9121 88.6139) (width 0.75) (layer F.Cu) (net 2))
 (segment (start 137.934 100.33) (end 137.934 94.592) (width 0.75) (layer F.Cu) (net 2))
 (segment (start 169.406 96.7691) (end 169.406 100.33) (width 0.75) (layer B.Cu) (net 2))
 (segment (start 161.2508 88.6139) (end 169.406 96.7691) (width 0.75) (layer B.Cu) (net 2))
 (segment (start 160.4285 88.6139) (end 161.2508 88.6139) (width 0.75) (layer B.Cu) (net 2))
 (segment (start 139.7 100.33) (end 137.934 100.33) (width 0.75) (layer F.Cu) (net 2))
 (segment (start 167.64 100.33) (end 169.406 100.33) (width 0.75) (layer B.Cu) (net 2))
 (via (at 158.9154 92.1162) (size 0.7) (layers F.Cu B.Cu) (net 1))
 (segment (start 165.6382 97.5542) (end 165.874 97.79) (width 0.75) (layer B.Cu) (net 1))
 (segment (start 157.7158 97.5542) (end 165.6382 97.5542) (width 0.75) (layer B.Cu) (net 1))
 (segment (start 154.94 100.33) (end 157.7158 97.5542) (width 0.75) (layer B.Cu) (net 1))
 (segment (start 167.64 97.79) (end 165.874 97.79) (width 0.75) (layer B.Cu) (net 1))
 (segment (start 157.9627 91.1635) (end 158.9154 92.1162) (width 0.75) (layer B.Cu) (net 1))
 (segment (start 141.4388 91.1635) (end 157.9627 91.1635) (width 0.75) (layer B.Cu) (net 1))
 (segment (start 139.7 92.9023) (end 141.4388 91.1635) (width 0.75) (layer B.Cu) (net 1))
 (segment (start 139.7 97.79) (end 139.7 92.9023) (width 0.75) (layer B.Cu) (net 1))
 (segment (start 163.5798 92.1162) (end 158.9154 92.1162) (width 0.75) (layer F.Cu) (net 1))
 (segment (start 167.64 96.1764) (end 163.5798 92.1162) (width 0.75) (layer F.Cu) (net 1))
 (segment (start 167.64 97.79) (end 167.64 96.1764) (width 0.75) (layer F.Cu) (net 1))
 (segment (start 142.1943 102.1417) (end 141.466 102.87) (width 0.75) (layer B.Cu) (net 7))
 (segment (start 148.0483 102.1417) (end 142.1943 102.1417) (width 0.75) (layer B.Cu) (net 7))
 (segment (start 149.86 100.33) (end 148.0483 102.1417) (width 0.75) (layer B.Cu) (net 7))
 (segment (start 139.7 102.87) (end 141.466 102.87) (width 0.75) (layer B.Cu) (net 7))
 (segment (start 147.95 98.43) (end 147.32 98.43) (width 0.75) (layer F.Cu) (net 39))
 (segment (start 152.4 93.98) (end 147.95 98.43) (width 0.75) (layer F.Cu) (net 39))
 (segment (start 147.32 100.33) (end 147.32 98.43) (width 0.75) (layer F.Cu) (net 39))
 (segment (start 134.62 113.03) (end 139.7 107.95) (width 0.75) (layer B.Cu) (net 5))
 (segment (start 134.62 113.15) (end 134.62 113.03) (width 0.75) (layer B.Cu) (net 5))
 (segment (start 172.72 84.0699) (end 172.72 95.13) (width 0.75) (layer F.Cu) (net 5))
 (segment (start 168.2567 79.6066) (end 172.72 84.0699) (width 0.75) (layer F.Cu) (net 5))
 (segment (start 138.5645 79.6066) (end 168.2567 79.6066) (width 0.75) (layer F.Cu) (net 5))
 (segment (start 136.9089 81.2622) (end 138.5645 79.6066) (width 0.75) (layer F.Cu) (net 5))
 (segment (start 136.9089 105.1589) (end 136.9089 81.2622) (width 0.75) (layer F.Cu) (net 5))
 (segment (start 139.7 107.95) (end 136.9089 105.1589) (width 0.75) (layer F.Cu) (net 5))
 (segment (start 172.72 102.87) (end 167.64 107.95) (width 0.75) (layer F.Cu) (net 5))
 (segment (start 172.72 95.13) (end 172.72 102.87) (width 0.75) (layer F.Cu) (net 5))
 (segment (start 164.0615 82.7815) (end 162.56 81.28) (width 0.75) (layer F.Cu) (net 17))
 (segment (start 164.0615 87.2619) (end 164.0615 82.7815) (width 0.75) (layer F.Cu) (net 17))
 (segment (start 161.6876 89.6358) (end 164.0615 87.2619) (width 0.75) (layer F.Cu) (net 17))
 (segment (start 149.1242 89.6358) (end 161.6876 89.6358) (width 0.75) (layer F.Cu) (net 17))
 (segment (start 144.78 93.98) (end 149.1242 89.6358) (width 0.75) (layer F.Cu) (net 17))
 (segment (start 165.1 87.638) (end 165.1 81.28) (width 0.75) (layer F.Cu) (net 18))
 (segment (start 162.1019 90.6361) (end 165.1 87.638) (width 0.75) (layer F.Cu) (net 18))
 (segment (start 150.6639 90.6361) (end 162.1019 90.6361) (width 0.75) (layer F.Cu) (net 18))
 (segment (start 147.32 93.98) (end 150.6639 90.6361) (width 0.75) (layer F.Cu) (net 18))
 (segment (start 143.3473 85.2527) (end 147.32 81.28) (width 0.75) (layer B.Cu) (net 11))
 (segment (start 143.3473 87.2951) (end 143.3473 85.2527) (width 0.75) (layer B.Cu) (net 11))
 (segment (start 146.2152 90.163) (end 143.3473 87.2951) (width 0.75) (layer B.Cu) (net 11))
 (segment (start 158.743 90.163) (end 146.2152 90.163) (width 0.75) (layer B.Cu) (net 11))
 (segment (start 162.56 93.98) (end 158.743 90.163) (width 0.75) (layer B.Cu) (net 11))
 (segment (start 151.508 79.632) (end 149.86 81.28) (width 0.75) (layer B.Cu) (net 12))
 (segment (start 168.2503 79.632) (end 151.508 79.632) (width 0.75) (layer B.Cu) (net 12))
 (segment (start 169.1535 80.5352) (end 168.2503 79.632) (width 0.75) (layer B.Cu) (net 12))
 (segment (start 169.1535 82.0803) (end 169.1535 80.5352) (width 0.75) (layer B.Cu) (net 12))
 (segment (start 164.8738 86.36) (end 169.1535 82.0803) (width 0.75) (layer B.Cu) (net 12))
 (segment (start 162.56 86.36) (end 164.8738 86.36) (width 0.75) (layer B.Cu) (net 12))
 (segment (start 160.02 86.36) (end 160.02 81.28) (width 0.75) (layer F.Cu) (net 16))
 (segment (start 157.48 86.36) (end 157.48 81.28) (width 0.75) (layer F.Cu) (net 15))
 (segment (start 152.4 86.36) (end 152.4 81.28) (width 0.75) (layer F.Cu) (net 13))
 (segment (start 149.86 86.36) (end 154.94 81.28) (width 0.75) (layer B.Cu) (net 14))
 (segment (start 147.32 83.82) (end 144.78 81.28) (width 0.75) (layer F.Cu) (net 10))
 (segment (start 147.32 86.36) (end 147.32 83.82) (width 0.75) (layer F.Cu) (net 10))
 (segment (start 143.23 84.036) (end 142.24 83.046) (width 0.75) (layer F.Cu) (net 9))
 (segment (start 143.23 86.36) (end 143.23 84.036) (width 0.75) (layer F.Cu) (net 9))
 (segment (start 144.78 86.36) (end 143.23 86.36) (width 0.75) (layer F.Cu) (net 9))
 (segment (start 142.24 81.28) (end 142.24 83.046) (width 0.75) (layer F.Cu) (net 9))
 (segment (start 143.127 128.653) (end 144.78 127) (width 0.75) (layer F.Cu) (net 29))
 (segment (start 139.0296 128.653) (end 143.127 128.653) (width 0.75) (layer F.Cu) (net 29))
 (segment (start 138.1639 127.7873) (end 139.0296 128.653) (width 0.75) (layer F.Cu) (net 29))
 (segment (start 138.1639 126.2582) (end 138.1639 127.7873) (width 0.75) (layer F.Cu) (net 29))
 (segment (start 142.5021 121.92) (end 138.1639 126.2582) (width 0.75) (layer F.Cu) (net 29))
 (segment (start 144.78 121.92) (end 142.5021 121.92) (width 0.75) (layer F.Cu) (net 29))
 (segment (start 147.32 121.92) (end 142.24 127) (width 0.75) (layer F.Cu) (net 30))
 (segment (start 160.02 124.46) (end 160.02 127) (width 0.75) (layer F.Cu) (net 23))
 (segment (start 162.56 121.92) (end 160.02 124.46) (width 0.75) (layer F.Cu) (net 23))
 (via (at 164.5449 123.8115) (size 0.7) (layers F.Cu B.Cu) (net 24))
 (segment (start 164.9902 123.3662) (end 164.5449 123.8115) (width 0.75) (layer F.Cu) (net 24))
 (segment (start 164.9902 115.1802) (end 164.9902 123.3662) (width 0.75) (layer F.Cu) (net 24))
 (segment (start 164.11 114.3) (end 164.9902 115.1802) (width 0.75) (layer F.Cu) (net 24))
 (segment (start 159.3064 125.1736) (end 157.48 127) (width 0.75) (layer B.Cu) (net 24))
 (segment (start 163.1828 125.1736) (end 159.3064 125.1736) (width 0.75) (layer B.Cu) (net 24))
 (segment (start 164.5449 123.8115) (end 163.1828 125.1736) (width 0.75) (layer B.Cu) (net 24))
 (segment (start 162.56 114.3) (end 164.11 114.3) (width 0.75) (layer F.Cu) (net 24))
 (via (at 148.4783 129.9106) (size 0.7) (layers F.Cu B.Cu) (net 28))
 (segment (start 167.5234 129.9106) (end 148.4783 129.9106) (width 0.75) (layer B.Cu) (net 28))
 (segment (start 169.129 128.305) (end 167.5234 129.9106) (width 0.75) (layer B.Cu) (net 28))
 (segment (start 169.129 123.2454) (end 169.129 128.305) (width 0.75) (layer B.Cu) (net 28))
 (segment (start 160.1836 114.3) (end 169.129 123.2454) (width 0.75) (layer B.Cu) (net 28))
 (segment (start 160.02 114.3) (end 160.1836 114.3) (width 0.75) (layer B.Cu) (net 28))
 (segment (start 147.3337 128.766) (end 147.32 128.766) (width 0.75) (layer F.Cu) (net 28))
 (segment (start 148.4783 129.9106) (end 147.3337 128.766) (width 0.75) (layer F.Cu) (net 28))
 (segment (start 147.32 127) (end 147.32 128.766) (width 0.75) (layer F.Cu) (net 28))
 (via (at 170.241 122.5442) (size 0.7) (layers F.Cu B.Cu) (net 27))
 (segment (start 170.241 119.5691) (end 170.241 122.5442) (width 0.75) (layer B.Cu) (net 27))
 (segment (start 163.1535 112.4816) (end 170.241 119.5691) (width 0.75) (layer B.Cu) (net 27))
 (segment (start 159.2984 112.4816) (end 163.1535 112.4816) (width 0.75) (layer B.Cu) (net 27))
 (segment (start 157.48 114.3) (end 159.2984 112.4816) (width 0.75) (layer B.Cu) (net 27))
 (segment (start 170.241 128.6533) (end 170.241 122.5442) (width 0.75) (layer F.Cu) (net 27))
 (segment (start 169.1837 129.7106) (end 170.241 128.6533) (width 0.75) (layer F.Cu) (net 27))
 (segment (start 152.5706 129.7106) (end 169.1837 129.7106) (width 0.75) (layer F.Cu) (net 27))
 (segment (start 149.86 127) (end 152.5706 129.7106) (width 0.75) (layer F.Cu) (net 27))
 (via (at 152.4 117.2675) (size 0.7) (layers F.Cu B.Cu) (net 25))
 (segment (start 160.311 117.2675) (end 152.4 117.2675) (width 0.75) (layer B.Cu) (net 25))
 (segment (start 164.0099 120.9664) (end 160.311 117.2675) (width 0.75) (layer B.Cu) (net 25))
 (segment (start 164.0099 122.9205) (end 164.0099 120.9664) (width 0.75) (layer B.Cu) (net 25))
 (segment (start 162.7572 124.1732) (end 164.0099 122.9205) (width 0.75) (layer B.Cu) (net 25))
 (segment (start 157.7668 124.1732) (end 162.7572 124.1732) (width 0.75) (layer B.Cu) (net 25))
 (segment (start 154.94 127) (end 157.7668 124.1732) (width 0.75) (layer B.Cu) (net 25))
 (segment (start 152.4 114.3) (end 152.4 117.2675) (width 0.75) (layer F.Cu) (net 25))
 (segment (start 154.0879 128.6879) (end 152.4 127) (width 0.75) (layer F.Cu) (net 26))
 (segment (start 168.7469 128.6879) (end 154.0879 128.6879) (width 0.75) (layer F.Cu) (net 26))
 (segment (start 169.129 128.3058) (end 168.7469 128.6879) (width 0.75) (layer F.Cu) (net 26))
 (segment (start 169.129 117.9029) (end 169.129 128.3058) (width 0.75) (layer F.Cu) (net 26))
 (segment (start 163.7394 112.5133) (end 169.129 117.9029) (width 0.75) (layer F.Cu) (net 26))
 (segment (start 151.6467 112.5133) (end 163.7394 112.5133) (width 0.75) (layer F.Cu) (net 26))
 (segment (start 149.86 114.3) (end 151.6467 112.5133) (width 0.75) (layer F.Cu) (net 26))
 (segment (start 162.56 127) (end 162.56 125.234) (width 0.75) (layer F.Cu) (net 22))
 (segment (start 162.56 124.3818) (end 162.56 125.234) (width 0.75) (layer F.Cu) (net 22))
 (segment (start 163.9898 122.952) (end 162.56 124.3818) (width 0.75) (layer F.Cu) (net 22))
 (segment (start 163.9898 120.9497) (end 163.9898 122.952) (width 0.75) (layer F.Cu) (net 22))
 (segment (start 162.1618 119.1217) (end 163.9898 120.9497) (width 0.75) (layer F.Cu) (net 22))
 (segment (start 152.1417 119.1217) (end 162.1618 119.1217) (width 0.75) (layer F.Cu) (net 22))
 (segment (start 147.32 114.3) (end 152.1417 119.1217) (width 0.75) (layer F.Cu) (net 22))
 (segment (start 146.6146 116.1346) (end 144.78 114.3) (width 0.75) (layer B.Cu) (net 21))
 (segment (start 160.5927 116.1346) (end 146.6146 116.1346) (width 0.75) (layer B.Cu) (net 21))
 (segment (start 165.5452 121.0871) (end 160.5927 116.1346) (width 0.75) (layer B.Cu) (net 21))
 (segment (start 165.5452 124.7888) (end 165.5452 121.0871) (width 0.75) (layer B.Cu) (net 21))
 (segment (start 165.1 125.234) (end 165.5452 124.7888) (width 0.75) (layer B.Cu) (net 21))
 (segment (start 165.1 127) (end 165.1 125.234) (width 0.75) (layer B.Cu) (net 21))
 (segment (start 142.355 78.625) (end 139.7 81.28) (width 0.75) (layer B.Cu) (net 8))
 (segment (start 171.215 78.625) (end 142.355 78.625) (width 0.75) (layer B.Cu) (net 8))
 (segment (start 172.72 80.13) (end 171.215 78.625) (width 0.75) (layer B.Cu) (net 8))
 (segment (start 165.9937 128.6463) (end 167.64 127) (width 0.75) (layer B.Cu) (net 20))
 (segment (start 135.1163 128.6463) (end 165.9937 128.6463) (width 0.75) (layer B.Cu) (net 20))
 (segment (start 134.62 128.15) (end 135.1163 128.6463) (width 0.75) (layer B.Cu) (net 20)))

